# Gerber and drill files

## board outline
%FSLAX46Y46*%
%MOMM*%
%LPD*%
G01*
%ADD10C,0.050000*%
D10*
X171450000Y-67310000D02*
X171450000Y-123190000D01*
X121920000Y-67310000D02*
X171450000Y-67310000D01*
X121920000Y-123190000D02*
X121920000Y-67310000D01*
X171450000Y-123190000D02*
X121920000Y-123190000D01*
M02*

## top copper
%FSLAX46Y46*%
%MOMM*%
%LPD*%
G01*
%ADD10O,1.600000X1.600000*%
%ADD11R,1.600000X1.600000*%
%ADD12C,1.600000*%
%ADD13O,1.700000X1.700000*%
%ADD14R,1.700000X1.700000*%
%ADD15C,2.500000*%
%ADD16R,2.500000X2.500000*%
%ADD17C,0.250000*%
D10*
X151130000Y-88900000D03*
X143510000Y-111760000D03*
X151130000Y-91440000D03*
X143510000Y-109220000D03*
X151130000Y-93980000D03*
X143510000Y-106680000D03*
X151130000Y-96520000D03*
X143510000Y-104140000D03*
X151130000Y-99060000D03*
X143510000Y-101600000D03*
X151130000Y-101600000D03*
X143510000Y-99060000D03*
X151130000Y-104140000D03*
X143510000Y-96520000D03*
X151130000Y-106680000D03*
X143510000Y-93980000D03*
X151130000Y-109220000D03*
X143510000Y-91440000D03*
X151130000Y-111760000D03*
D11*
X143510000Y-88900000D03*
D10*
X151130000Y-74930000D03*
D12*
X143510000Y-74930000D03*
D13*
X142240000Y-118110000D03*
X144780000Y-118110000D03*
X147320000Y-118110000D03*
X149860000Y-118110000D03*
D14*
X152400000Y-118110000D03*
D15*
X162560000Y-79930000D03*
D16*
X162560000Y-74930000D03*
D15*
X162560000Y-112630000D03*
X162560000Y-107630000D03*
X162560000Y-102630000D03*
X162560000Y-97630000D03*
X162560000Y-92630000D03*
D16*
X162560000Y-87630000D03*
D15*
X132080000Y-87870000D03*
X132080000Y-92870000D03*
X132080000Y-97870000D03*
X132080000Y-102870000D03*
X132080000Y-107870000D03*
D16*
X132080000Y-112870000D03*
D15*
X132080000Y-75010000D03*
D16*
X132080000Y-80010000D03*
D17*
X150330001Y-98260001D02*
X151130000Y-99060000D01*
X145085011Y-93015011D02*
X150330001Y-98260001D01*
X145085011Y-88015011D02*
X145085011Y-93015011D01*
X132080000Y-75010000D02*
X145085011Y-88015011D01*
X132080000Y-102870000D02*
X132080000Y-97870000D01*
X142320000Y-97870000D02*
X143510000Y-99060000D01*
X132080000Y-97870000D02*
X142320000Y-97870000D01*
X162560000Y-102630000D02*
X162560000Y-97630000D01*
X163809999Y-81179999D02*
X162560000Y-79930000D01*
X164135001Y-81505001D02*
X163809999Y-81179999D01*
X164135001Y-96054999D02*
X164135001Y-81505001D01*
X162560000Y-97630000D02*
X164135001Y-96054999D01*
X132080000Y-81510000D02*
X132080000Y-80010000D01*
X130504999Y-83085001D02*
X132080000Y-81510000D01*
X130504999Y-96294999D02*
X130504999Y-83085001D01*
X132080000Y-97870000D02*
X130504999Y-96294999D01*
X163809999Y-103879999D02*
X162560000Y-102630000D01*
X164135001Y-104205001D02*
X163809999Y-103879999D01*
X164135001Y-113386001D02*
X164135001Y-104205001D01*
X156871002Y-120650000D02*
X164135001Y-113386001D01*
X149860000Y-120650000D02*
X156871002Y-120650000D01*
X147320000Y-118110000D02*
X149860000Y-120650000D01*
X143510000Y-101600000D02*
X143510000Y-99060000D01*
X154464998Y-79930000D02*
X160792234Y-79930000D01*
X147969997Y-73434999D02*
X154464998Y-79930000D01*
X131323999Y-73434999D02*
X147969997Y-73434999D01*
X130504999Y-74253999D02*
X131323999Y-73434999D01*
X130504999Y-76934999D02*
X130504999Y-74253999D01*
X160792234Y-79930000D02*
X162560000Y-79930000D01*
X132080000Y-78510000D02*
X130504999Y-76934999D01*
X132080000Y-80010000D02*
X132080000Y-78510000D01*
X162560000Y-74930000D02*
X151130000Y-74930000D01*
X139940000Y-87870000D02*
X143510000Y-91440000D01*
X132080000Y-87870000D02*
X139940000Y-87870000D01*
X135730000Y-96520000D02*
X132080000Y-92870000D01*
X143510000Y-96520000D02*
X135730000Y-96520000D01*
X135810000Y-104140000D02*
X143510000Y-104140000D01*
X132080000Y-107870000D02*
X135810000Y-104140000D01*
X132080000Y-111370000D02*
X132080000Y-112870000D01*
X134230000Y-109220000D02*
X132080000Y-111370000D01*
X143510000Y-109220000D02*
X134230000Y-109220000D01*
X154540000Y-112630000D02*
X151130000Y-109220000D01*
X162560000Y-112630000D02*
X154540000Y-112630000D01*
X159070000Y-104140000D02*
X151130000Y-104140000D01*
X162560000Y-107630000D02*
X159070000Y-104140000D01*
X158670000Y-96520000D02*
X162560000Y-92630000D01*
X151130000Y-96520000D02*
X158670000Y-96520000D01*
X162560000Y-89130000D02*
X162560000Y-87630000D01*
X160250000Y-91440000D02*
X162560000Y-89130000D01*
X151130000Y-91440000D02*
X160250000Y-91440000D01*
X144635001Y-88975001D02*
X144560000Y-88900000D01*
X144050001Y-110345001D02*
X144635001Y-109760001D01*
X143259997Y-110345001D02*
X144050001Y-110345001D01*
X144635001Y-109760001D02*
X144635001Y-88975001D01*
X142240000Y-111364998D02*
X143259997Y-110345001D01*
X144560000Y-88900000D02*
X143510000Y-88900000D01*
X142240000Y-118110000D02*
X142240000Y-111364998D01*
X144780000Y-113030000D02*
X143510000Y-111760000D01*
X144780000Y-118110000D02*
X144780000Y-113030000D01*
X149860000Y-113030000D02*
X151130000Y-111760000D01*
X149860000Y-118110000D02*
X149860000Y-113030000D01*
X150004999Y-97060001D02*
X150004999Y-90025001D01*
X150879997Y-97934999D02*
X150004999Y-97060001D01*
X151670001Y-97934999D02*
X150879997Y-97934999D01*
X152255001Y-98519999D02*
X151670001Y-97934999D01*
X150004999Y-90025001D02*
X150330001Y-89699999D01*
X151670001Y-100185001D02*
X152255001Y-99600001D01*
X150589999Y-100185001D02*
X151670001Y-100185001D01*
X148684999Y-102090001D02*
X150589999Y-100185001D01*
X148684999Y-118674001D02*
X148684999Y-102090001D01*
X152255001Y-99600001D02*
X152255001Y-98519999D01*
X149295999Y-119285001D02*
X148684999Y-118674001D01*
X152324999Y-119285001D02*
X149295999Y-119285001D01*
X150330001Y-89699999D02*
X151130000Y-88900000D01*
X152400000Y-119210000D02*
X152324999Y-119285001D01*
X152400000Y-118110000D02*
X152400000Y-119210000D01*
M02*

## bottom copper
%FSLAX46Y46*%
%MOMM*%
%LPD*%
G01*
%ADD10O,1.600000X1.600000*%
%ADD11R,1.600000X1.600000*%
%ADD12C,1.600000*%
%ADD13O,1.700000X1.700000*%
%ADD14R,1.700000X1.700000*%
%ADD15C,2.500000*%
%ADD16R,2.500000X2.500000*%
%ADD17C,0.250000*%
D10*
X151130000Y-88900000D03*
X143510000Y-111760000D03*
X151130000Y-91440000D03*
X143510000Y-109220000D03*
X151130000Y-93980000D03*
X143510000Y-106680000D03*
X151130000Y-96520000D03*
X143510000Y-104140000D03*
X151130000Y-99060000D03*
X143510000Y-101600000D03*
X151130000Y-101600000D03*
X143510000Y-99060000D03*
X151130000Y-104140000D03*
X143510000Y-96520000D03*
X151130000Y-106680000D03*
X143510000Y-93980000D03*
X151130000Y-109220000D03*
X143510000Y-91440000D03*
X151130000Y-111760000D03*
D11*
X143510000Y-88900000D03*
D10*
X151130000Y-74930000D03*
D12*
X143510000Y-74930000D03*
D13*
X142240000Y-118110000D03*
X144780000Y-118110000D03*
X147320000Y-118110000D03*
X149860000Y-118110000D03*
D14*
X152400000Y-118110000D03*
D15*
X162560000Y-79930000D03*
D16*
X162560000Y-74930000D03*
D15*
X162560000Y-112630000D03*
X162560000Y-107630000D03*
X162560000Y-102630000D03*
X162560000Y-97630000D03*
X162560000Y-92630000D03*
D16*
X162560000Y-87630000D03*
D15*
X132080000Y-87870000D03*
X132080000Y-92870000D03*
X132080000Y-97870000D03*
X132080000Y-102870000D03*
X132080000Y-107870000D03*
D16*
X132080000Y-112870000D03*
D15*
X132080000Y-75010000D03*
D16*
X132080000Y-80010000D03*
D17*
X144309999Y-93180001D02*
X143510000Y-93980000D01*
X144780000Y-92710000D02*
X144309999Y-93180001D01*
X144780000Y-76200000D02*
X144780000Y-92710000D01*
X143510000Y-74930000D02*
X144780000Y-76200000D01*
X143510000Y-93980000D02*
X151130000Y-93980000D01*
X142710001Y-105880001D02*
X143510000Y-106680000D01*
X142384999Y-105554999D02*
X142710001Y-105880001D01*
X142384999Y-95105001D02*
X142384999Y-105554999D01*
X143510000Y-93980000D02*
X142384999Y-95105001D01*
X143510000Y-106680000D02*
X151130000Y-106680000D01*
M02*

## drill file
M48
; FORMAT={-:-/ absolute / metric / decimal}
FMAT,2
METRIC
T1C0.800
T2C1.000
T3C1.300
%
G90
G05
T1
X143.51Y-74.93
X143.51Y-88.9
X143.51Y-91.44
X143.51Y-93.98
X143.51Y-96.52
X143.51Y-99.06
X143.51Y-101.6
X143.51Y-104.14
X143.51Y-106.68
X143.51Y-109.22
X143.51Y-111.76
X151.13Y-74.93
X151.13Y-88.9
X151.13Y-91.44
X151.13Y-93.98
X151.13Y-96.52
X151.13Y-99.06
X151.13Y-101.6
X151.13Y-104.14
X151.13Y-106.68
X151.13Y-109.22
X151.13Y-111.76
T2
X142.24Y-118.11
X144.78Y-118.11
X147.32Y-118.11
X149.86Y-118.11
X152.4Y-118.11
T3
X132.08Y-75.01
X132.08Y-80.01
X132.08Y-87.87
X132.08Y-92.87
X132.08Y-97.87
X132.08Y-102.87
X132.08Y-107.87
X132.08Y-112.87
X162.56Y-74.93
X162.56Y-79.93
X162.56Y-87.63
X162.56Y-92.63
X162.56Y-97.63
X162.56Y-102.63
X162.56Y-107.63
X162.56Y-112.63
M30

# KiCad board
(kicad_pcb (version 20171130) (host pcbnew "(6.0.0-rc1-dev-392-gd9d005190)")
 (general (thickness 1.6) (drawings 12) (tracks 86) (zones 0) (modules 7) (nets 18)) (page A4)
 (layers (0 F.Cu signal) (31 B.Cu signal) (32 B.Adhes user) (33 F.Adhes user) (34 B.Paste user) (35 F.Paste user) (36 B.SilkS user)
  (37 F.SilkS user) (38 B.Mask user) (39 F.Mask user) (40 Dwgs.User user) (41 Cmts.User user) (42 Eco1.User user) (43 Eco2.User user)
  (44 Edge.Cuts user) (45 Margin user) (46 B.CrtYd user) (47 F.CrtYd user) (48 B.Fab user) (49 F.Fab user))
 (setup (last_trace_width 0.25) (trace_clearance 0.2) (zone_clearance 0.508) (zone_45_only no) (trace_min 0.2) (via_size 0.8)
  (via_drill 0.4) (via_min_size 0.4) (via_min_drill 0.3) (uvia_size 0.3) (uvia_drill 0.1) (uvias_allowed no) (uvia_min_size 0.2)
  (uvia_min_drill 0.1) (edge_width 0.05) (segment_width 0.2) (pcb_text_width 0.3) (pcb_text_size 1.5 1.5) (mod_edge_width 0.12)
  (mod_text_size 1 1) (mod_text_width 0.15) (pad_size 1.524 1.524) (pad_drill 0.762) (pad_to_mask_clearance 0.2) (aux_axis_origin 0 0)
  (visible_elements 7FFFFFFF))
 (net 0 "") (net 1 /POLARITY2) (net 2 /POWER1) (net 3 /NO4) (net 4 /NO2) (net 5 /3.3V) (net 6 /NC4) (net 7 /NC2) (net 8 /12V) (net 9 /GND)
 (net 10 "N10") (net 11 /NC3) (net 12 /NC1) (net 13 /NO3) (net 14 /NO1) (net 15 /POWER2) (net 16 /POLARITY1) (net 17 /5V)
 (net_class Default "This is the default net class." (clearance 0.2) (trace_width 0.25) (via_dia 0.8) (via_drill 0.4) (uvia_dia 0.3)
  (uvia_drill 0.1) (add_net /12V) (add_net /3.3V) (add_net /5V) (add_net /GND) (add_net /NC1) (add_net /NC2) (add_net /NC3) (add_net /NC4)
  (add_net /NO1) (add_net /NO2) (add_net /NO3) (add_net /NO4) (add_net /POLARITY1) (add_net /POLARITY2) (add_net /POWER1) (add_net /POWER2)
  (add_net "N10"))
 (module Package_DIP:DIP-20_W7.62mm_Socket (layer F.Cu) (at 143.51 88.9)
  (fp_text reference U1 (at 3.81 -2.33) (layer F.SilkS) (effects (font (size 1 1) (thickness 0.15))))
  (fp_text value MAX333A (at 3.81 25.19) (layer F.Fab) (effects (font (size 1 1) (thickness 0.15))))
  (pad 20 thru_hole oval (at 7.62 0) (size 1.6 1.6) (drill 0.8) (layers *.Cu *.Mask) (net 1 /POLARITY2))
  (pad 10 thru_hole oval (at 0 22.86) (size 1.6 1.6) (drill 0.8) (layers *.Cu *.Mask) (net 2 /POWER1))
  (pad 19 thru_hole oval (at 7.62 2.54) (size 1.6 1.6) (drill 0.8) (layers *.Cu *.Mask) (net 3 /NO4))
  (pad 9 thru_hole oval (at 0 20.32) (size 1.6 1.6) (drill 0.8) (layers *.Cu *.Mask) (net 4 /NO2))
  (pad 18 thru_hole oval (at 7.62 5.08) (size 1.6 1.6) (drill 0.8) (layers *.Cu *.Mask) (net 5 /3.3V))
  (pad 8 thru_hole oval (at 0 17.78) (size 1.6 1.6) (drill 0.8) (layers *.Cu *.Mask) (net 5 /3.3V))
  (pad 17 thru_hole oval (at 7.62 7.62) (size 1.6 1.6) (drill 0.8) (layers *.Cu *.Mask) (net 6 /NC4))
  (pad 7 thru_hole oval (at 0 15.24) (size 1.6 1.6) (drill 0.8) (layers *.Cu *.Mask) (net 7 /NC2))
  (pad 16 thru_hole oval (at 7.62 10.16) (size 1.6 1.6) (drill 0.8) (layers *.Cu *.Mask) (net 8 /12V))
  (pad 6 thru_hole oval (at 0 12.7) (size 1.6 1.6) (drill 0.8) (layers *.Cu *.Mask) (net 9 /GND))
  (pad 15 thru_hole oval (at 7.62 12.7) (size 1.6 1.6) (drill 0.8) (layers *.Cu *.Mask) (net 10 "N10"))
  (pad 5 thru_hole oval (at 0 10.16) (size 1.6 1.6) (drill 0.8) (layers *.Cu *.Mask) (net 9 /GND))
  (pad 14 thru_hole oval (at 7.62 15.24) (size 1.6 1.6) (drill 0.8) (layers *.Cu *.Mask) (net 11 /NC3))
  (pad 4 thru_hole oval (at 0 7.62) (size 1.6 1.6) (drill 0.8) (layers *.Cu *.Mask) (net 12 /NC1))
  (pad 13 thru_hole oval (at 7.62 17.78) (size 1.6 1.6) (drill 0.8) (layers *.Cu *.Mask) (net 5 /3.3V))
  (pad 3 thru_hole oval (at 0 5.08) (size 1.6 1.6) (drill 0.8) (layers *.Cu *.Mask) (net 5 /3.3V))
  (pad 12 thru_hole oval (at 7.62 20.32) (size 1.6 1.6) (drill 0.8) (layers *.Cu *.Mask) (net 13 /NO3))
  (pad 2 thru_hole oval (at 0 2.54) (size 1.6 1.6) (drill 0.8) (layers *.Cu *.Mask) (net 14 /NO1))
  (pad 11 thru_hole oval (at 7.62 22.86) (size 1.6 1.6) (drill 0.8) (layers *.Cu *.Mask) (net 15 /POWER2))
  (pad 1 thru_hole rect (at 0 0) (size 1.6 1.6) (drill 0.8) (layers *.Cu *.Mask) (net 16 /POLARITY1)))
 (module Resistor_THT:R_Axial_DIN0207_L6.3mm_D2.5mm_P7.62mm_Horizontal (layer F.Cu) (at 143.51 74.93)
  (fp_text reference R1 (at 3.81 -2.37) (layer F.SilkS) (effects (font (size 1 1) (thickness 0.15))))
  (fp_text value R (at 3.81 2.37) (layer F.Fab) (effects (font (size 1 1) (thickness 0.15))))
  (pad 2 thru_hole oval (at 7.62 0) (size 1.6 1.6) (drill 0.8) (layers *.Cu *.Mask) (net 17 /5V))
  (pad 1 thru_hole circle (at 0 0) (size 1.6 1.6) (drill 0.8) (layers *.Cu *.Mask) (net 5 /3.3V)))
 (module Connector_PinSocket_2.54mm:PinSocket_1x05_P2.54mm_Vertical (layer F.Cu) (at 152.4 118.11 270)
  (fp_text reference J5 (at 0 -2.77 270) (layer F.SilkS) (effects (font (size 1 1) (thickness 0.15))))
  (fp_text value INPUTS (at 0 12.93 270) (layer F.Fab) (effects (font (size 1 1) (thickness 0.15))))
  (pad 5 thru_hole oval (at 0 10.16 270) (size 1.7 1.7) (drill 1) (layers *.Cu *.Mask) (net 16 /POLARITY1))
  (pad 4 thru_hole oval (at 0 7.62 270) (size 1.7 1.7) (drill 1) (layers *.Cu *.Mask) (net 2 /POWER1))
  (pad 3 thru_hole oval (at 0 5.08 270) (size 1.7 1.7) (drill 1) (layers *.Cu *.Mask) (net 9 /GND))
  (pad 2 thru_hole oval (at 0 2.54 270) (size 1.7 1.7) (drill 1) (layers *.Cu *.Mask) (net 15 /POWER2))
  (pad 1 thru_hole rect (at 0 0 270) (size 1.7 1.7) (drill 1) (layers *.Cu *.Mask) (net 1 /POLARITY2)))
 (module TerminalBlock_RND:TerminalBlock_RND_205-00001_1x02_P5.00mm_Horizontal (layer F.Cu) (at 162.56 74.93 270)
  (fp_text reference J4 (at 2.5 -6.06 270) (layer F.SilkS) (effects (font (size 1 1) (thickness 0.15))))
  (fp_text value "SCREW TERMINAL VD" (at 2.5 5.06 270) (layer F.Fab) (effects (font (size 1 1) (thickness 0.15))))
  (pad 2 thru_hole circle (at 5 0 270) (size 2.5 2.5) (drill 1.3) (layers *.Cu *.Mask) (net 9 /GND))
  (pad 1 thru_hole rect (at 0 0 270) (size 2.5 2.5) (drill 1.3) (layers *.Cu *.Mask) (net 17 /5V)))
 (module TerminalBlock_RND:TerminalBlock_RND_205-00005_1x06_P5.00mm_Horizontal (layer F.Cu) (at 162.56 87.63 270)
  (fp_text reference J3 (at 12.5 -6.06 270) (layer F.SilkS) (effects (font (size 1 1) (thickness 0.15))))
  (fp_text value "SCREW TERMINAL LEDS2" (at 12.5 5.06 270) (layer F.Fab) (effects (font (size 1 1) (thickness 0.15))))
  (pad 6 thru_hole circle (at 25 0 270) (size 2.5 2.5) (drill 1.3) (layers *.Cu *.Mask) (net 13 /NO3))
  (pad 5 thru_hole circle (at 20 0 270) (size 2.5 2.5) (drill 1.3) (layers *.Cu *.Mask) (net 11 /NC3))
  (pad 4 thru_hole circle (at 15 0 270) (size 2.5 2.5) (drill 1.3) (layers *.Cu *.Mask) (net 9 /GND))
  (pad 3 thru_hole circle (at 10 0 270) (size 2.5 2.5) (drill 1.3) (layers *.Cu *.Mask) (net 9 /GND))
  (pad 2 thru_hole circle (at 5 0 270) (size 2.5 2.5) (drill 1.3) (layers *.Cu *.Mask) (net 6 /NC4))
  (pad 1 thru_hole rect (at 0 0 270) (size 2.5 2.5) (drill 1.3) (layers *.Cu *.Mask) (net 3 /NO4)))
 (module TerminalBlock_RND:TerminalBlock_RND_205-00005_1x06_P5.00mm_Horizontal (layer F.Cu) (at 132.08 112.87 90)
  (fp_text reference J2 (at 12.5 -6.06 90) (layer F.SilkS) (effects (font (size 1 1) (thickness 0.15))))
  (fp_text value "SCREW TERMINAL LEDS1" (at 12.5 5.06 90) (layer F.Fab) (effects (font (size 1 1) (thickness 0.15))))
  (pad 6 thru_hole circle (at 25 0 90) (size 2.5 2.5) (drill 1.3) (layers *.Cu *.Mask) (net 14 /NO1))
  (pad 5 thru_hole circle (at 20 0 90) (size 2.5 2.5) (drill 1.3) (layers *.Cu *.Mask) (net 12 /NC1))
  (pad 4 thru_hole circle (at 15 0 90) (size 2.5 2.5) (drill 1.3) (layers *.Cu *.Mask) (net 9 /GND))
  (pad 3 thru_hole circle (at 10 0 90) (size 2.5 2.5) (drill 1.3) (layers *.Cu *.Mask) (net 9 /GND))
  (pad 2 thru_hole circle (at 5 0 90) (size 2.5 2.5) (drill 1.3) (layers *.Cu *.Mask) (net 7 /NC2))
  (pad 1 thru_hole rect (at 0 0 90) (size 2.5 2.5) (drill 1.3) (layers *.Cu *.Mask) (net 4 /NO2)))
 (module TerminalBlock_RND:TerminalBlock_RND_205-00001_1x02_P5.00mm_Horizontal (layer F.Cu) (at 132.08 80.01 90)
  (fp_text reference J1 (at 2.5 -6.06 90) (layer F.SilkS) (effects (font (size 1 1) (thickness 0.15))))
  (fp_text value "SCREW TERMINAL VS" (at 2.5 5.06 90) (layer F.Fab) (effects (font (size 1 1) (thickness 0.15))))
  (pad 2 thru_hole circle (at 5 0 90) (size 2.5 2.5) (drill 1.3) (layers *.Cu *.Mask) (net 8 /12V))
  (pad 1 thru_hole rect (at 0 0 90) (size 2.5 2.5) (drill 1.3) (layers *.Cu *.Mask) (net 9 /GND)))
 (gr_line (start 171.45 67.31) (end 171.45 123.19) (layer Edge.Cuts) (width 0.05))
 (gr_line (start 121.92 67.31) (end 171.45 67.31) (layer Edge.Cuts) (width 0.05))
 (gr_line (start 121.92 123.19) (end 121.92 67.31) (layer Edge.Cuts) (width 0.05))
 (gr_line (start 171.45 123.19) (end 121.92 123.19) (layer Edge.Cuts) (width 0.05))
 (segment (start 150.330001 98.260001) (end 151.13 99.06) (width 0.25) (layer F.Cu) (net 8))
 (segment (start 145.085011 93.015011) (end 150.330001 98.260001) (width 0.25) (layer F.Cu) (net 8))
 (segment (start 145.085011 88.015011) (end 145.085011 93.015011) (width 0.25) (layer F.Cu) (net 8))
 (segment (start 132.08 75.01) (end 145.085011 88.015011) (width 0.25) (layer F.Cu) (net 8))
 (segment (start 132.08 102.87) (end 132.08 97.87) (width 0.25) (layer F.Cu) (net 9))
 (segment (start 142.32 97.87) (end 143.51 99.06) (width 0.25) (layer F.Cu) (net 9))
 (segment (start 132.08 97.87) (end 142.32 97.87) (width 0.25) (layer F.Cu) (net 9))
 (segment (start 162.56 102.63) (end 162.56 97.63) (width 0.25) (layer F.Cu) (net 9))
 (segment (start 163.809999 81.179999) (end 162.56 79.93) (width 0.25) (layer F.Cu) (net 9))
 (segment (start 164.135001 81.505001) (end 163.809999 81.179999) (width 0.25) (layer F.Cu) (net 9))
 (segment (start 164.135001 96.054999) (end 164.135001 81.505001) (width 0.25) (layer F.Cu) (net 9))
 (segment (start 162.56 97.63) (end 164.135001 96.054999) (width 0.25) (layer F.Cu) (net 9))
 (segment (start 132.08 81.51) (end 132.08 80.01) (width 0.25) (layer F.Cu) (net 9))
 (segment (start 130.504999 83.085001) (end 132.08 81.51) (width 0.25) (layer F.Cu) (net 9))
 (segment (start 130.504999 96.294999) (end 130.504999 83.085001) (width 0.25) (layer F.Cu) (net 9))
 (segment (start 132.08 97.87) (end 130.504999 96.294999) (width 0.25) (layer F.Cu) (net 9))
 (segment (start 163.809999 103.879999) (end 162.56 102.63) (width 0.25) (layer F.Cu) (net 9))
 (segment (start 164.135001 104.205001) (end 163.809999 103.879999) (width 0.25) (layer F.Cu) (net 9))
 (segment (start 164.135001 113.386001) (end 164.135001 104.205001) (width 0.25) (layer F.Cu) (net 9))
 (segment (start 156.871002 120.65) (end 164.135001 113.386001) (width 0.25) (layer F.Cu) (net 9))
 (segment (start 149.86 120.65) (end 156.871002 120.65) (width 0.25) (layer F.Cu) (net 9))
 (segment (start 147.32 118.11) (end 149.86 120.65) (width 0.25) (layer F.Cu) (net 9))
 (segment (start 143.51 101.6) (end 143.51 99.06) (width 0.25) (layer F.Cu) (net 9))
 (segment (start 154.464998 79.93) (end 160.792234 79.93) (width 0.25) (layer F.Cu) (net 9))
 (segment (start 147.969997 73.434999) (end 154.464998 79.93) (width 0.25) (layer F.Cu) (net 9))
 (segment (start 131.323999 73.434999) (end 147.969997 73.434999) (width 0.25) (layer F.Cu) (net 9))
 (segment (start 130.504999 74.253999) (end 131.323999 73.434999) (width 0.25) (layer F.Cu) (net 9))
 (segment (start 130.504999 76.934999) (end 130.504999 74.253999) (width 0.25) (layer F.Cu) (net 9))
 (segment (start 160.792234 79.93) (end 162.56 79.93) (width 0.25) (layer F.Cu) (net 9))
 (segment (start 132.08 78.51) (end 130.504999 76.934999) (width 0.25) (layer F.Cu) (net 9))
 (segment (start 132.08 80.01) (end 132.08 78.51) (width 0.25) (layer F.Cu) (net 9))
 (segment (start 162.56 74.93) (end 151.13 74.93) (width 0.25) (layer F.Cu) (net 17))
 (segment (start 144.309999 93.180001) (end 143.51 93.98) (width 0.25) (layer B.Cu) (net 5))
 (segment (start 144.78 92.71) (end 144.309999 93.180001) (width 0.25) (layer B.Cu) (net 5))
 (segment (start 144.78 76.2) (end 144.78 92.71) (width 0.25) (layer B.Cu) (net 5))
 (segment (start 143.51 74.93) (end 144.78 76.2) (width 0.25) (layer B.Cu) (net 5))
 (segment (start 143.51 93.98) (end 151.13 93.98) (width 0.25) (layer B.Cu) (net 5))
 (segment (start 142.710001 105.880001) (end 143.51 106.68) (width 0.25) (layer B.Cu) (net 5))
 (segment (start 142.384999 105.554999) (end 142.710001 105.880001) (width 0.25) (layer B.Cu) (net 5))
 (segment (start 142.384999 95.105001) (end 142.384999 105.554999) (width 0.25) (layer B.Cu) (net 5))
 (segment (start 143.51 93.98) (end 142.384999 95.105001) (width 0.25) (layer B.Cu) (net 5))
 (segment (start 143.51 106.68) (end 151.13 106.68) (width 0.25) (layer B.Cu) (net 5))
 (segment (start 139.94 87.87) (end 143.51 91.44) (width 0.25) (layer F.Cu) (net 14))
 (segment (start 132.08 87.87) (end 139.94 87.87) (width 0.25) (layer F.Cu) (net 14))
 (segment (start 135.73 96.52) (end 132.08 92.87) (width 0.25) (layer F.Cu) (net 12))
 (segment (start 143.51 96.52) (end 135.73 96.52) (width 0.25) (layer F.Cu) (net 12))
 (segment (start 135.81 104.14) (end 143.51 104.14) (width 0.25) (layer F.Cu) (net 7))
 (segment (start 132.08 107.87) (end 135.81 104.14) (width 0.25) (layer F.Cu) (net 7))
 (segment (start 132.08 111.37) (end 132.08 112.87) (width 0.25) (layer F.Cu) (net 4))
 (segment (start 134.23 109.22) (end 132.08 111.37) (width 0.25) (layer F.Cu) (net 4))
 (segment (start 143.51 109.22) (end 134.23 109.22) (width 0.25) (layer F.Cu) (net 4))
 (segment (start 154.54 112.63) (end 151.13 109.22) (width 0.25) (layer F.Cu) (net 13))
 (segment (start 162.56 112.63) (end 154.54 112.63) (width 0.25) (layer F.Cu) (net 13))
 (segment (start 159.07 104.14) (end 151.13 104.14) (width 0.25) (layer F.Cu) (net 11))
 (segment (start 162.56 107.63) (end 159.07 104.14) (width 0.25) (layer F.Cu) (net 11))
 (segment (start 158.67 96.52) (end 162.56 92.63) (width 0.25) (layer F.Cu) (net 6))
 (segment (start 151.13 96.52) (end 158.67 96.52) (width 0.25) (layer F.Cu) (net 6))
 (segment (start 162.56 89.13) (end 162.56 87.63) (width 0.25) (layer F.Cu) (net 3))
 (segment (start 160.25 91.44) (end 162.56 89.13) (width 0.25) (layer F.Cu) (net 3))
 (segment (start 151.13 91.44) (end 160.25 91.44) (width 0.25) (layer F.Cu) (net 3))
 (segment (start 144.635001 88.975001) (end 144.56 88.9) (width 0.25) (layer F.Cu) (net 16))
 (segment (start 144.050001 110.345001) (end 144.635001 109.760001) (width 0.25) (layer F.Cu) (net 16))
 (segment (start 143.259997 110.345001) (end 144.050001 110.345001) (width 0.25) (layer F.Cu) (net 16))
 (segment (start 144.635001 109.760001) (end 144.635001 88.975001) (width 0.25) (layer F.Cu) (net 16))
 (segment (start 142.24 111.364998) (end 143.259997 110.345001) (width 0.25) (layer F.Cu) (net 16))
 (segment (start 144.56 88.9) (end 143.51 88.9) (width 0.25) (layer F.Cu) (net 16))
 (segment (start 142.24 118.11) (end 142.24 111.364998) (width 0.25) (layer F.Cu) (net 16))
 (segment (start 144.78 113.03) (end 143.51 111.76) (width 0.25) (layer F.Cu) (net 2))
 (segment (start 144.78 118.11) (end 144.78 113.03) (width 0.25) (layer F.Cu) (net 2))
 (segment (start 149.86 113.03) (end 151.13 111.76) (width 0.25) (layer F.Cu) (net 15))
 (segment (start 149.86 118.11) (end 149.86 113.03) (width 0.25) (layer F.Cu) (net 15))
 (segment (start 150.004999 97.060001) (end 150.004999 90.025001) (width 0.25) (layer F.Cu) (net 1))
 (segment (start 150.879997 97.934999) (end 150.004999 97.060001) (width 0.25) (layer F.Cu) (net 1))
 (segment (start 151.670001 97.934999) (end 150.879997 97.934999) (width 0.25) (layer F.Cu) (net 1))
 (segment (start 152.255001 98.519999) (end 151.670001 97.934999) (width 0.25) (layer F.Cu) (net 1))
 (segment (start 150.004999 90.025001) (end 150.330001 89.699999) (width 0.25) (layer F.Cu) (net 1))
 (segment (start 151.670001 100.185001) (end 152.255001 99.600001) (width 0.25) (layer F.Cu) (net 1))
 (segment (start 150.589999 100.185001) (end 151.670001 100.185001) (width 0.25) (layer F.Cu) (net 1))
 (segment (start 148.684999 102.090001) (end 150.589999 100.185001) (width 0.25) (layer F.Cu) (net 1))
 (segment (start 148.684999 118.674001) (end 148.684999 102.090001) (width 0.25) (layer F.Cu) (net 1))
 (segment (start 152.255001 99.600001) (end 152.255001 98.519999) (width 0.25) (layer F.Cu) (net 1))
 (segment (start 149.295999 119.285001) (end 148.684999 118.674001) (width 0.25) (layer F.Cu) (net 1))
 (segment (start 152.324999 119.285001) (end 149.295999 119.285001) (width 0.25) (layer F.Cu) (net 1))
 (segment (start 150.330001 89.699999) (end 151.13 88.9) (width 0.25) (layer F.Cu) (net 1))
 (segment (start 152.4 119.21) (end 152.324999 119.285001) (width 0.25) (layer F.Cu) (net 1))
 (segment (start 152.4 118.11) (end 152.4 119.21) (width 0.25) (layer F.Cu) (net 1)))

